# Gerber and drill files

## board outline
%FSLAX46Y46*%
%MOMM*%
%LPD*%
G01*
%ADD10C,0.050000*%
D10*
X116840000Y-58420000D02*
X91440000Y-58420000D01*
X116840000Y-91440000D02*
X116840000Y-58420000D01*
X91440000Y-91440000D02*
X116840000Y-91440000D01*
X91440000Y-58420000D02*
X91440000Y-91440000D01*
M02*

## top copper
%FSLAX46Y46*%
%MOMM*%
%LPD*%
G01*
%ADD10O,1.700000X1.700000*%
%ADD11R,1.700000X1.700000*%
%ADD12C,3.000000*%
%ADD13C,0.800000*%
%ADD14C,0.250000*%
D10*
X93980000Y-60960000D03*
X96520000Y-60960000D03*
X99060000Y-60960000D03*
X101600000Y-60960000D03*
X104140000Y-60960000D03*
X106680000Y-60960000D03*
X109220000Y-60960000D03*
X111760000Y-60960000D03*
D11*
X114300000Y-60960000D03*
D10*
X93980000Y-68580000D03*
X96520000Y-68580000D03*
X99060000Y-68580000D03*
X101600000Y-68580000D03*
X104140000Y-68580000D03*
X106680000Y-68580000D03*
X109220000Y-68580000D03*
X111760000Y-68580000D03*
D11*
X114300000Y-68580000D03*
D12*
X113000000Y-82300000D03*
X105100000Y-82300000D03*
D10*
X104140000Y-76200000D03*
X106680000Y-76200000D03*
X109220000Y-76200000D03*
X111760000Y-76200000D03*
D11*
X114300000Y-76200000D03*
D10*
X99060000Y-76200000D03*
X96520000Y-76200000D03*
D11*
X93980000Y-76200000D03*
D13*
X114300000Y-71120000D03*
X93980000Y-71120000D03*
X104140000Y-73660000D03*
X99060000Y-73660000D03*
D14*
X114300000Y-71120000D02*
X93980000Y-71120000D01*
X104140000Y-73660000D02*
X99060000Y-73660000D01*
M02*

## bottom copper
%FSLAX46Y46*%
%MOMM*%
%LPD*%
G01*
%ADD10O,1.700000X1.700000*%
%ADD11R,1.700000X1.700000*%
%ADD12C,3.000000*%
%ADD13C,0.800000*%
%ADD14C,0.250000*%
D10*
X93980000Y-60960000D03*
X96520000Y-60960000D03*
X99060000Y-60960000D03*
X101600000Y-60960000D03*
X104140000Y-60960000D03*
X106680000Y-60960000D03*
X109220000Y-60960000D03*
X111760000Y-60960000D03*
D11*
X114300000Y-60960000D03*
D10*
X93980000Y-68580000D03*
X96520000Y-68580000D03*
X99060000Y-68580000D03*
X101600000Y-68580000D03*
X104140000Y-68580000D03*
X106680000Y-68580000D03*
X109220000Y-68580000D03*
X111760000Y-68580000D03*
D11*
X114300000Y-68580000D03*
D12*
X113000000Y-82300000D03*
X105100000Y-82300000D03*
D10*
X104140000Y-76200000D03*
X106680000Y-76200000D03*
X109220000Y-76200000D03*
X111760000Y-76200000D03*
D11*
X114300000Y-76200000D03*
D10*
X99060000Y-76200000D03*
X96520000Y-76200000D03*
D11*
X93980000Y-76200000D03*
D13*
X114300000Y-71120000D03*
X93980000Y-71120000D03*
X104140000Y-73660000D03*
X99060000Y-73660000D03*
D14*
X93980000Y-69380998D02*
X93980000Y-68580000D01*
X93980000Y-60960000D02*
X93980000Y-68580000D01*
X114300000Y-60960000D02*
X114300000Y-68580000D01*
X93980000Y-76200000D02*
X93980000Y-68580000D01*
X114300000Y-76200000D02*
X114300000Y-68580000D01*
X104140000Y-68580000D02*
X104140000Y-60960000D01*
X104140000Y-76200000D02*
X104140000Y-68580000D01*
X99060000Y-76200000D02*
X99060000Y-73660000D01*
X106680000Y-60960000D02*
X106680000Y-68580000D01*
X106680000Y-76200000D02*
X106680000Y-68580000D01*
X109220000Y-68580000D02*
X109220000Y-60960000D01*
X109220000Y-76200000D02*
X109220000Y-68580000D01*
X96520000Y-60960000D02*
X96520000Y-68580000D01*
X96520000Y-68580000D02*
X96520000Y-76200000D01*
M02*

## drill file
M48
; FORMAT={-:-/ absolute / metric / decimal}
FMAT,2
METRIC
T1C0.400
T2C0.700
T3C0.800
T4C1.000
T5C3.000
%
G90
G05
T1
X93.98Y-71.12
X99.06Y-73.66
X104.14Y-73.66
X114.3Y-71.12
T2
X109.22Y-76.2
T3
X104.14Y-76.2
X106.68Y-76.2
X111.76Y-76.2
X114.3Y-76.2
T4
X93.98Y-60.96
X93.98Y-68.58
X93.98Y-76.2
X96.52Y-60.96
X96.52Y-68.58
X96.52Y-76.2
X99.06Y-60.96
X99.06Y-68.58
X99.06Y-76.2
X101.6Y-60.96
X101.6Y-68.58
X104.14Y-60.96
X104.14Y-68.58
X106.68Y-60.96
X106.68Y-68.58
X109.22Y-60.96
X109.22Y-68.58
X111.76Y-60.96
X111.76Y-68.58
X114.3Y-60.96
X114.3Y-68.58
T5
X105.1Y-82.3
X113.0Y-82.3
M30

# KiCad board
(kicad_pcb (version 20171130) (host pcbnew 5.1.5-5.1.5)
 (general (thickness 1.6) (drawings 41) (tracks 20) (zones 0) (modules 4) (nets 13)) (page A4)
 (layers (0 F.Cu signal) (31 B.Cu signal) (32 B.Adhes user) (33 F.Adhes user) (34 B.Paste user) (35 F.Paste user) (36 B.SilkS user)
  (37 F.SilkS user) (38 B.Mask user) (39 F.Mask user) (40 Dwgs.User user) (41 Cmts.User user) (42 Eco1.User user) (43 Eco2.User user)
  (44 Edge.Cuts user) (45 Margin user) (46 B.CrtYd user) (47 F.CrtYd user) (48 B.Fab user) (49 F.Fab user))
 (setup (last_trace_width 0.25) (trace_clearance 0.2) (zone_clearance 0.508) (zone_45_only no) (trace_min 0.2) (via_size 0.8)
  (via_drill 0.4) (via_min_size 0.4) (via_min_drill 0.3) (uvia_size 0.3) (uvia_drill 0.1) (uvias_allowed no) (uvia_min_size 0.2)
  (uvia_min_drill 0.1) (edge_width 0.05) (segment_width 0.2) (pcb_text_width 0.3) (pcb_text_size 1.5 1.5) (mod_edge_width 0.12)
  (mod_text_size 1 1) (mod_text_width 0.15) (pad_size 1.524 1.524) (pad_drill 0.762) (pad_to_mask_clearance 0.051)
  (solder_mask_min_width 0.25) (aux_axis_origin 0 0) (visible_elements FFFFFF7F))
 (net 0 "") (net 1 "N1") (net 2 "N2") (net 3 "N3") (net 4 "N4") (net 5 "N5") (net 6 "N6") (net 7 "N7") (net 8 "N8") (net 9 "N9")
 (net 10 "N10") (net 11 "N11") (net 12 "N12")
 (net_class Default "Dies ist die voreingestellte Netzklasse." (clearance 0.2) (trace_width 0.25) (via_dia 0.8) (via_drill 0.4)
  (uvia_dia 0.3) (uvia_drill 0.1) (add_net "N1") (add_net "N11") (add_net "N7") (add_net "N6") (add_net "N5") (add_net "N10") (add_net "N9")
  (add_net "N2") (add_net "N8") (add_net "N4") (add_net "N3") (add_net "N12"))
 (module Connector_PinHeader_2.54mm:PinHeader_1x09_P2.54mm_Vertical (layer B.Cu) (at 114.3 60.96 90)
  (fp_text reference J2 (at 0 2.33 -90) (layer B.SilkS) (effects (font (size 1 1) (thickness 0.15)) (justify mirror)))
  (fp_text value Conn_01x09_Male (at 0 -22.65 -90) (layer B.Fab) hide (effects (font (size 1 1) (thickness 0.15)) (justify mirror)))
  (pad 9 thru_hole oval (at 0 -20.32 90) (size 1.7 1.7) (drill 1) (layers *.Cu *.Mask) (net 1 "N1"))
  (pad 8 thru_hole oval (at 0 -17.78 90) (size 1.7 1.7) (drill 1) (layers *.Cu *.Mask) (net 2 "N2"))
  (pad 7 thru_hole oval (at 0 -15.24 90) (size 1.7 1.7) (drill 1) (layers *.Cu *.Mask) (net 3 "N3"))
  (pad 6 thru_hole oval (at 0 -12.7 90) (size 1.7 1.7) (drill 1) (layers *.Cu *.Mask) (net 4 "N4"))
  (pad 5 thru_hole oval (at 0 -10.16 90) (size 1.7 1.7) (drill 1) (layers *.Cu *.Mask) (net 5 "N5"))
  (pad 4 thru_hole oval (at 0 -7.62 90) (size 1.7 1.7) (drill 1) (layers *.Cu *.Mask) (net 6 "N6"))
  (pad 3 thru_hole oval (at 0 -5.08 90) (size 1.7 1.7) (drill 1) (layers *.Cu *.Mask) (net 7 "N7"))
  (pad 2 thru_hole oval (at 0 -2.54 90) (size 1.7 1.7) (drill 1) (layers *.Cu *.Mask) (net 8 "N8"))
  (pad 1 thru_hole rect (at 0 0 90) (size 1.7 1.7) (drill 1) (layers *.Cu *.Mask) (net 1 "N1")))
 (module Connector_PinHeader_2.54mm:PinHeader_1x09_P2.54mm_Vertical (layer B.Cu) (at 114.3 68.58 90)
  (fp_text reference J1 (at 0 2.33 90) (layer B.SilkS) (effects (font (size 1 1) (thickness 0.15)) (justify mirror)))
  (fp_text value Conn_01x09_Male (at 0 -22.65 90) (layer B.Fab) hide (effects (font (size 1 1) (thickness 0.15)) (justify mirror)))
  (pad 9 thru_hole oval (at 0 -20.32 90) (size 1.7 1.7) (drill 1) (layers *.Cu *.Mask) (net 1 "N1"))
  (pad 8 thru_hole oval (at 0 -17.78 90) (size 1.7 1.7) (drill 1) (layers *.Cu *.Mask) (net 2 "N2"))
  (pad 7 thru_hole oval (at 0 -15.24 90) (size 1.7 1.7) (drill 1) (layers *.Cu *.Mask) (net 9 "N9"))
  (pad 6 thru_hole oval (at 0 -12.7 90) (size 1.7 1.7) (drill 1) (layers *.Cu *.Mask) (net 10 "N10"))
  (pad 5 thru_hole oval (at 0 -10.16 90) (size 1.7 1.7) (drill 1) (layers *.Cu *.Mask) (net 5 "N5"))
  (pad 4 thru_hole oval (at 0 -7.62 90) (size 1.7 1.7) (drill 1) (layers *.Cu *.Mask) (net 6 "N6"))
  (pad 3 thru_hole oval (at 0 -5.08 90) (size 1.7 1.7) (drill 1) (layers *.Cu *.Mask) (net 7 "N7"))
  (pad 2 thru_hole oval (at 0 -2.54 90) (size 1.7 1.7) (drill 1) (layers *.Cu *.Mask) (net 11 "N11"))
  (pad 1 thru_hole rect (at 0 0 90) (size 1.7 1.7) (drill 1) (layers *.Cu *.Mask) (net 1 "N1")))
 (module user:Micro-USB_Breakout (layer F.Cu) (at 114.3 76.2 270)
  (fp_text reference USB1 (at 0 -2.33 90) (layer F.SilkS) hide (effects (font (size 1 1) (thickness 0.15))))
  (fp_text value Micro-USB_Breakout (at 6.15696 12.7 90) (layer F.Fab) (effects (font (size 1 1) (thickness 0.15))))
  (pad 7 thru_hole circle (at 6.1 1.3 270) (size 3 3) (drill 3) (layers *.Cu *.Mask))
  (pad 6 thru_hole circle (at 6.1 9.2 270) (size 3 3) (drill 3) (layers *.Cu *.Mask))
  (pad 5 thru_hole oval (at 0 10.16 270) (size 1.7 1.7) (drill 0.8) (layers *.Cu *.Mask) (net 5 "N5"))
  (pad 4 thru_hole oval (at 0 7.62 270) (size 1.7 1.7) (drill 0.8) (layers *.Cu *.Mask) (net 6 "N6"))
  (pad 3 thru_hole oval (at 0 5.08 270) (size 1.7 1.7) (drill 0.7) (layers *.Cu *.Mask) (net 7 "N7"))
  (pad 2 thru_hole oval (at 0 2.54 270) (size 1.7 1.7) (drill 0.8) (layers *.Cu *.Mask) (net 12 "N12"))
  (pad 1 thru_hole rect (at 0 0 270) (size 1.7 1.7) (drill 0.8) (layers *.Cu *.Mask) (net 1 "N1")))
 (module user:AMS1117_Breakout (layer F.Cu) (at 93.98 76.2 90)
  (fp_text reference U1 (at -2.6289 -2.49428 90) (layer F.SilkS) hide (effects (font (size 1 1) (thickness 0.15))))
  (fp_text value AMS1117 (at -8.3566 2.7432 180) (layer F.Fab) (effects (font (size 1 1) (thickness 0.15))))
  (pad 3 thru_hole oval (at 0 5.08 90) (size 1.7 1.7) (drill 1) (layers *.Cu *.Mask) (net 5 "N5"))
  (pad 2 thru_hole oval (at 0 2.54 90) (size 1.7 1.7) (drill 1) (layers *.Cu *.Mask) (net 2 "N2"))
  (pad 1 thru_hole rect (at 0 0 90) (size 1.7 1.7) (drill 1) (layers *.Cu *.Mask) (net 1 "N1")))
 (gr_line (start 116.84 58.42) (end 91.44 58.42) (layer Edge.Cuts) (width 0.05))
 (gr_line (start 116.84 91.44) (end 116.84 58.42) (layer Edge.Cuts) (width 0.05))
 (gr_line (start 91.44 91.44) (end 116.84 91.44) (layer Edge.Cuts) (width 0.05))
 (gr_line (start 91.44 58.42) (end 91.44 91.44) (layer Edge.Cuts) (width 0.05))
 (segment (start 93.98 69.380998) (end 93.98 68.58) (width 0.25) (layer B.Cu) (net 1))
 (segment (start 93.98 60.96) (end 93.98 68.58) (width 0.25) (layer B.Cu) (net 1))
 (segment (start 114.3 60.96) (end 114.3 68.58) (width 0.25) (layer B.Cu) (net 1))
 (via (at 114.3 71.12) (size 0.8) (drill 0.4) (layers F.Cu B.Cu) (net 1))
 (via (at 93.98 71.12) (size 0.8) (drill 0.4) (layers F.Cu B.Cu) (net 1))
 (segment (start 114.3 71.12) (end 93.98 71.12) (width 0.25) (layer F.Cu) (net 1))
 (segment (start 93.98 76.2) (end 93.98 68.58) (width 0.25) (layer B.Cu) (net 1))
 (segment (start 114.3 76.2) (end 114.3 68.58) (width 0.25) (layer B.Cu) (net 1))
 (segment (start 104.14 68.58) (end 104.14 60.96) (width 0.25) (layer B.Cu) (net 5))
 (via (at 104.14 73.66) (size 0.8) (drill 0.4) (layers F.Cu B.Cu) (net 5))
 (segment (start 104.14 76.2) (end 104.14 68.58) (width 0.25) (layer B.Cu) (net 5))
 (segment (start 104.14 73.66) (end 99.06 73.66) (width 0.25) (layer F.Cu) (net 5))
 (via (at 99.06 73.66) (size 0.8) (drill 0.4) (layers F.Cu B.Cu) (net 5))
 (segment (start 99.06 76.2) (end 99.06 73.66) (width 0.25) (layer B.Cu) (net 5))
 (segment (start 106.68 60.96) (end 106.68 68.58) (width 0.25) (layer B.Cu) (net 6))
 (segment (start 106.68 76.2) (end 106.68 68.58) (width 0.25) (layer B.Cu) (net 6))
 (segment (start 109.22 68.58) (end 109.22 60.96) (width 0.25) (layer B.Cu) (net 7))
 (segment (start 109.22 76.2) (end 109.22 68.58) (width 0.25) (layer B.Cu) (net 7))
 (segment (start 96.52 60.96) (end 96.52 68.58) (width 0.25) (layer B.Cu) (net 2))
 (segment (start 96.52 68.58) (end 96.52 76.2) (width 0.25) (layer B.Cu) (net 2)))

